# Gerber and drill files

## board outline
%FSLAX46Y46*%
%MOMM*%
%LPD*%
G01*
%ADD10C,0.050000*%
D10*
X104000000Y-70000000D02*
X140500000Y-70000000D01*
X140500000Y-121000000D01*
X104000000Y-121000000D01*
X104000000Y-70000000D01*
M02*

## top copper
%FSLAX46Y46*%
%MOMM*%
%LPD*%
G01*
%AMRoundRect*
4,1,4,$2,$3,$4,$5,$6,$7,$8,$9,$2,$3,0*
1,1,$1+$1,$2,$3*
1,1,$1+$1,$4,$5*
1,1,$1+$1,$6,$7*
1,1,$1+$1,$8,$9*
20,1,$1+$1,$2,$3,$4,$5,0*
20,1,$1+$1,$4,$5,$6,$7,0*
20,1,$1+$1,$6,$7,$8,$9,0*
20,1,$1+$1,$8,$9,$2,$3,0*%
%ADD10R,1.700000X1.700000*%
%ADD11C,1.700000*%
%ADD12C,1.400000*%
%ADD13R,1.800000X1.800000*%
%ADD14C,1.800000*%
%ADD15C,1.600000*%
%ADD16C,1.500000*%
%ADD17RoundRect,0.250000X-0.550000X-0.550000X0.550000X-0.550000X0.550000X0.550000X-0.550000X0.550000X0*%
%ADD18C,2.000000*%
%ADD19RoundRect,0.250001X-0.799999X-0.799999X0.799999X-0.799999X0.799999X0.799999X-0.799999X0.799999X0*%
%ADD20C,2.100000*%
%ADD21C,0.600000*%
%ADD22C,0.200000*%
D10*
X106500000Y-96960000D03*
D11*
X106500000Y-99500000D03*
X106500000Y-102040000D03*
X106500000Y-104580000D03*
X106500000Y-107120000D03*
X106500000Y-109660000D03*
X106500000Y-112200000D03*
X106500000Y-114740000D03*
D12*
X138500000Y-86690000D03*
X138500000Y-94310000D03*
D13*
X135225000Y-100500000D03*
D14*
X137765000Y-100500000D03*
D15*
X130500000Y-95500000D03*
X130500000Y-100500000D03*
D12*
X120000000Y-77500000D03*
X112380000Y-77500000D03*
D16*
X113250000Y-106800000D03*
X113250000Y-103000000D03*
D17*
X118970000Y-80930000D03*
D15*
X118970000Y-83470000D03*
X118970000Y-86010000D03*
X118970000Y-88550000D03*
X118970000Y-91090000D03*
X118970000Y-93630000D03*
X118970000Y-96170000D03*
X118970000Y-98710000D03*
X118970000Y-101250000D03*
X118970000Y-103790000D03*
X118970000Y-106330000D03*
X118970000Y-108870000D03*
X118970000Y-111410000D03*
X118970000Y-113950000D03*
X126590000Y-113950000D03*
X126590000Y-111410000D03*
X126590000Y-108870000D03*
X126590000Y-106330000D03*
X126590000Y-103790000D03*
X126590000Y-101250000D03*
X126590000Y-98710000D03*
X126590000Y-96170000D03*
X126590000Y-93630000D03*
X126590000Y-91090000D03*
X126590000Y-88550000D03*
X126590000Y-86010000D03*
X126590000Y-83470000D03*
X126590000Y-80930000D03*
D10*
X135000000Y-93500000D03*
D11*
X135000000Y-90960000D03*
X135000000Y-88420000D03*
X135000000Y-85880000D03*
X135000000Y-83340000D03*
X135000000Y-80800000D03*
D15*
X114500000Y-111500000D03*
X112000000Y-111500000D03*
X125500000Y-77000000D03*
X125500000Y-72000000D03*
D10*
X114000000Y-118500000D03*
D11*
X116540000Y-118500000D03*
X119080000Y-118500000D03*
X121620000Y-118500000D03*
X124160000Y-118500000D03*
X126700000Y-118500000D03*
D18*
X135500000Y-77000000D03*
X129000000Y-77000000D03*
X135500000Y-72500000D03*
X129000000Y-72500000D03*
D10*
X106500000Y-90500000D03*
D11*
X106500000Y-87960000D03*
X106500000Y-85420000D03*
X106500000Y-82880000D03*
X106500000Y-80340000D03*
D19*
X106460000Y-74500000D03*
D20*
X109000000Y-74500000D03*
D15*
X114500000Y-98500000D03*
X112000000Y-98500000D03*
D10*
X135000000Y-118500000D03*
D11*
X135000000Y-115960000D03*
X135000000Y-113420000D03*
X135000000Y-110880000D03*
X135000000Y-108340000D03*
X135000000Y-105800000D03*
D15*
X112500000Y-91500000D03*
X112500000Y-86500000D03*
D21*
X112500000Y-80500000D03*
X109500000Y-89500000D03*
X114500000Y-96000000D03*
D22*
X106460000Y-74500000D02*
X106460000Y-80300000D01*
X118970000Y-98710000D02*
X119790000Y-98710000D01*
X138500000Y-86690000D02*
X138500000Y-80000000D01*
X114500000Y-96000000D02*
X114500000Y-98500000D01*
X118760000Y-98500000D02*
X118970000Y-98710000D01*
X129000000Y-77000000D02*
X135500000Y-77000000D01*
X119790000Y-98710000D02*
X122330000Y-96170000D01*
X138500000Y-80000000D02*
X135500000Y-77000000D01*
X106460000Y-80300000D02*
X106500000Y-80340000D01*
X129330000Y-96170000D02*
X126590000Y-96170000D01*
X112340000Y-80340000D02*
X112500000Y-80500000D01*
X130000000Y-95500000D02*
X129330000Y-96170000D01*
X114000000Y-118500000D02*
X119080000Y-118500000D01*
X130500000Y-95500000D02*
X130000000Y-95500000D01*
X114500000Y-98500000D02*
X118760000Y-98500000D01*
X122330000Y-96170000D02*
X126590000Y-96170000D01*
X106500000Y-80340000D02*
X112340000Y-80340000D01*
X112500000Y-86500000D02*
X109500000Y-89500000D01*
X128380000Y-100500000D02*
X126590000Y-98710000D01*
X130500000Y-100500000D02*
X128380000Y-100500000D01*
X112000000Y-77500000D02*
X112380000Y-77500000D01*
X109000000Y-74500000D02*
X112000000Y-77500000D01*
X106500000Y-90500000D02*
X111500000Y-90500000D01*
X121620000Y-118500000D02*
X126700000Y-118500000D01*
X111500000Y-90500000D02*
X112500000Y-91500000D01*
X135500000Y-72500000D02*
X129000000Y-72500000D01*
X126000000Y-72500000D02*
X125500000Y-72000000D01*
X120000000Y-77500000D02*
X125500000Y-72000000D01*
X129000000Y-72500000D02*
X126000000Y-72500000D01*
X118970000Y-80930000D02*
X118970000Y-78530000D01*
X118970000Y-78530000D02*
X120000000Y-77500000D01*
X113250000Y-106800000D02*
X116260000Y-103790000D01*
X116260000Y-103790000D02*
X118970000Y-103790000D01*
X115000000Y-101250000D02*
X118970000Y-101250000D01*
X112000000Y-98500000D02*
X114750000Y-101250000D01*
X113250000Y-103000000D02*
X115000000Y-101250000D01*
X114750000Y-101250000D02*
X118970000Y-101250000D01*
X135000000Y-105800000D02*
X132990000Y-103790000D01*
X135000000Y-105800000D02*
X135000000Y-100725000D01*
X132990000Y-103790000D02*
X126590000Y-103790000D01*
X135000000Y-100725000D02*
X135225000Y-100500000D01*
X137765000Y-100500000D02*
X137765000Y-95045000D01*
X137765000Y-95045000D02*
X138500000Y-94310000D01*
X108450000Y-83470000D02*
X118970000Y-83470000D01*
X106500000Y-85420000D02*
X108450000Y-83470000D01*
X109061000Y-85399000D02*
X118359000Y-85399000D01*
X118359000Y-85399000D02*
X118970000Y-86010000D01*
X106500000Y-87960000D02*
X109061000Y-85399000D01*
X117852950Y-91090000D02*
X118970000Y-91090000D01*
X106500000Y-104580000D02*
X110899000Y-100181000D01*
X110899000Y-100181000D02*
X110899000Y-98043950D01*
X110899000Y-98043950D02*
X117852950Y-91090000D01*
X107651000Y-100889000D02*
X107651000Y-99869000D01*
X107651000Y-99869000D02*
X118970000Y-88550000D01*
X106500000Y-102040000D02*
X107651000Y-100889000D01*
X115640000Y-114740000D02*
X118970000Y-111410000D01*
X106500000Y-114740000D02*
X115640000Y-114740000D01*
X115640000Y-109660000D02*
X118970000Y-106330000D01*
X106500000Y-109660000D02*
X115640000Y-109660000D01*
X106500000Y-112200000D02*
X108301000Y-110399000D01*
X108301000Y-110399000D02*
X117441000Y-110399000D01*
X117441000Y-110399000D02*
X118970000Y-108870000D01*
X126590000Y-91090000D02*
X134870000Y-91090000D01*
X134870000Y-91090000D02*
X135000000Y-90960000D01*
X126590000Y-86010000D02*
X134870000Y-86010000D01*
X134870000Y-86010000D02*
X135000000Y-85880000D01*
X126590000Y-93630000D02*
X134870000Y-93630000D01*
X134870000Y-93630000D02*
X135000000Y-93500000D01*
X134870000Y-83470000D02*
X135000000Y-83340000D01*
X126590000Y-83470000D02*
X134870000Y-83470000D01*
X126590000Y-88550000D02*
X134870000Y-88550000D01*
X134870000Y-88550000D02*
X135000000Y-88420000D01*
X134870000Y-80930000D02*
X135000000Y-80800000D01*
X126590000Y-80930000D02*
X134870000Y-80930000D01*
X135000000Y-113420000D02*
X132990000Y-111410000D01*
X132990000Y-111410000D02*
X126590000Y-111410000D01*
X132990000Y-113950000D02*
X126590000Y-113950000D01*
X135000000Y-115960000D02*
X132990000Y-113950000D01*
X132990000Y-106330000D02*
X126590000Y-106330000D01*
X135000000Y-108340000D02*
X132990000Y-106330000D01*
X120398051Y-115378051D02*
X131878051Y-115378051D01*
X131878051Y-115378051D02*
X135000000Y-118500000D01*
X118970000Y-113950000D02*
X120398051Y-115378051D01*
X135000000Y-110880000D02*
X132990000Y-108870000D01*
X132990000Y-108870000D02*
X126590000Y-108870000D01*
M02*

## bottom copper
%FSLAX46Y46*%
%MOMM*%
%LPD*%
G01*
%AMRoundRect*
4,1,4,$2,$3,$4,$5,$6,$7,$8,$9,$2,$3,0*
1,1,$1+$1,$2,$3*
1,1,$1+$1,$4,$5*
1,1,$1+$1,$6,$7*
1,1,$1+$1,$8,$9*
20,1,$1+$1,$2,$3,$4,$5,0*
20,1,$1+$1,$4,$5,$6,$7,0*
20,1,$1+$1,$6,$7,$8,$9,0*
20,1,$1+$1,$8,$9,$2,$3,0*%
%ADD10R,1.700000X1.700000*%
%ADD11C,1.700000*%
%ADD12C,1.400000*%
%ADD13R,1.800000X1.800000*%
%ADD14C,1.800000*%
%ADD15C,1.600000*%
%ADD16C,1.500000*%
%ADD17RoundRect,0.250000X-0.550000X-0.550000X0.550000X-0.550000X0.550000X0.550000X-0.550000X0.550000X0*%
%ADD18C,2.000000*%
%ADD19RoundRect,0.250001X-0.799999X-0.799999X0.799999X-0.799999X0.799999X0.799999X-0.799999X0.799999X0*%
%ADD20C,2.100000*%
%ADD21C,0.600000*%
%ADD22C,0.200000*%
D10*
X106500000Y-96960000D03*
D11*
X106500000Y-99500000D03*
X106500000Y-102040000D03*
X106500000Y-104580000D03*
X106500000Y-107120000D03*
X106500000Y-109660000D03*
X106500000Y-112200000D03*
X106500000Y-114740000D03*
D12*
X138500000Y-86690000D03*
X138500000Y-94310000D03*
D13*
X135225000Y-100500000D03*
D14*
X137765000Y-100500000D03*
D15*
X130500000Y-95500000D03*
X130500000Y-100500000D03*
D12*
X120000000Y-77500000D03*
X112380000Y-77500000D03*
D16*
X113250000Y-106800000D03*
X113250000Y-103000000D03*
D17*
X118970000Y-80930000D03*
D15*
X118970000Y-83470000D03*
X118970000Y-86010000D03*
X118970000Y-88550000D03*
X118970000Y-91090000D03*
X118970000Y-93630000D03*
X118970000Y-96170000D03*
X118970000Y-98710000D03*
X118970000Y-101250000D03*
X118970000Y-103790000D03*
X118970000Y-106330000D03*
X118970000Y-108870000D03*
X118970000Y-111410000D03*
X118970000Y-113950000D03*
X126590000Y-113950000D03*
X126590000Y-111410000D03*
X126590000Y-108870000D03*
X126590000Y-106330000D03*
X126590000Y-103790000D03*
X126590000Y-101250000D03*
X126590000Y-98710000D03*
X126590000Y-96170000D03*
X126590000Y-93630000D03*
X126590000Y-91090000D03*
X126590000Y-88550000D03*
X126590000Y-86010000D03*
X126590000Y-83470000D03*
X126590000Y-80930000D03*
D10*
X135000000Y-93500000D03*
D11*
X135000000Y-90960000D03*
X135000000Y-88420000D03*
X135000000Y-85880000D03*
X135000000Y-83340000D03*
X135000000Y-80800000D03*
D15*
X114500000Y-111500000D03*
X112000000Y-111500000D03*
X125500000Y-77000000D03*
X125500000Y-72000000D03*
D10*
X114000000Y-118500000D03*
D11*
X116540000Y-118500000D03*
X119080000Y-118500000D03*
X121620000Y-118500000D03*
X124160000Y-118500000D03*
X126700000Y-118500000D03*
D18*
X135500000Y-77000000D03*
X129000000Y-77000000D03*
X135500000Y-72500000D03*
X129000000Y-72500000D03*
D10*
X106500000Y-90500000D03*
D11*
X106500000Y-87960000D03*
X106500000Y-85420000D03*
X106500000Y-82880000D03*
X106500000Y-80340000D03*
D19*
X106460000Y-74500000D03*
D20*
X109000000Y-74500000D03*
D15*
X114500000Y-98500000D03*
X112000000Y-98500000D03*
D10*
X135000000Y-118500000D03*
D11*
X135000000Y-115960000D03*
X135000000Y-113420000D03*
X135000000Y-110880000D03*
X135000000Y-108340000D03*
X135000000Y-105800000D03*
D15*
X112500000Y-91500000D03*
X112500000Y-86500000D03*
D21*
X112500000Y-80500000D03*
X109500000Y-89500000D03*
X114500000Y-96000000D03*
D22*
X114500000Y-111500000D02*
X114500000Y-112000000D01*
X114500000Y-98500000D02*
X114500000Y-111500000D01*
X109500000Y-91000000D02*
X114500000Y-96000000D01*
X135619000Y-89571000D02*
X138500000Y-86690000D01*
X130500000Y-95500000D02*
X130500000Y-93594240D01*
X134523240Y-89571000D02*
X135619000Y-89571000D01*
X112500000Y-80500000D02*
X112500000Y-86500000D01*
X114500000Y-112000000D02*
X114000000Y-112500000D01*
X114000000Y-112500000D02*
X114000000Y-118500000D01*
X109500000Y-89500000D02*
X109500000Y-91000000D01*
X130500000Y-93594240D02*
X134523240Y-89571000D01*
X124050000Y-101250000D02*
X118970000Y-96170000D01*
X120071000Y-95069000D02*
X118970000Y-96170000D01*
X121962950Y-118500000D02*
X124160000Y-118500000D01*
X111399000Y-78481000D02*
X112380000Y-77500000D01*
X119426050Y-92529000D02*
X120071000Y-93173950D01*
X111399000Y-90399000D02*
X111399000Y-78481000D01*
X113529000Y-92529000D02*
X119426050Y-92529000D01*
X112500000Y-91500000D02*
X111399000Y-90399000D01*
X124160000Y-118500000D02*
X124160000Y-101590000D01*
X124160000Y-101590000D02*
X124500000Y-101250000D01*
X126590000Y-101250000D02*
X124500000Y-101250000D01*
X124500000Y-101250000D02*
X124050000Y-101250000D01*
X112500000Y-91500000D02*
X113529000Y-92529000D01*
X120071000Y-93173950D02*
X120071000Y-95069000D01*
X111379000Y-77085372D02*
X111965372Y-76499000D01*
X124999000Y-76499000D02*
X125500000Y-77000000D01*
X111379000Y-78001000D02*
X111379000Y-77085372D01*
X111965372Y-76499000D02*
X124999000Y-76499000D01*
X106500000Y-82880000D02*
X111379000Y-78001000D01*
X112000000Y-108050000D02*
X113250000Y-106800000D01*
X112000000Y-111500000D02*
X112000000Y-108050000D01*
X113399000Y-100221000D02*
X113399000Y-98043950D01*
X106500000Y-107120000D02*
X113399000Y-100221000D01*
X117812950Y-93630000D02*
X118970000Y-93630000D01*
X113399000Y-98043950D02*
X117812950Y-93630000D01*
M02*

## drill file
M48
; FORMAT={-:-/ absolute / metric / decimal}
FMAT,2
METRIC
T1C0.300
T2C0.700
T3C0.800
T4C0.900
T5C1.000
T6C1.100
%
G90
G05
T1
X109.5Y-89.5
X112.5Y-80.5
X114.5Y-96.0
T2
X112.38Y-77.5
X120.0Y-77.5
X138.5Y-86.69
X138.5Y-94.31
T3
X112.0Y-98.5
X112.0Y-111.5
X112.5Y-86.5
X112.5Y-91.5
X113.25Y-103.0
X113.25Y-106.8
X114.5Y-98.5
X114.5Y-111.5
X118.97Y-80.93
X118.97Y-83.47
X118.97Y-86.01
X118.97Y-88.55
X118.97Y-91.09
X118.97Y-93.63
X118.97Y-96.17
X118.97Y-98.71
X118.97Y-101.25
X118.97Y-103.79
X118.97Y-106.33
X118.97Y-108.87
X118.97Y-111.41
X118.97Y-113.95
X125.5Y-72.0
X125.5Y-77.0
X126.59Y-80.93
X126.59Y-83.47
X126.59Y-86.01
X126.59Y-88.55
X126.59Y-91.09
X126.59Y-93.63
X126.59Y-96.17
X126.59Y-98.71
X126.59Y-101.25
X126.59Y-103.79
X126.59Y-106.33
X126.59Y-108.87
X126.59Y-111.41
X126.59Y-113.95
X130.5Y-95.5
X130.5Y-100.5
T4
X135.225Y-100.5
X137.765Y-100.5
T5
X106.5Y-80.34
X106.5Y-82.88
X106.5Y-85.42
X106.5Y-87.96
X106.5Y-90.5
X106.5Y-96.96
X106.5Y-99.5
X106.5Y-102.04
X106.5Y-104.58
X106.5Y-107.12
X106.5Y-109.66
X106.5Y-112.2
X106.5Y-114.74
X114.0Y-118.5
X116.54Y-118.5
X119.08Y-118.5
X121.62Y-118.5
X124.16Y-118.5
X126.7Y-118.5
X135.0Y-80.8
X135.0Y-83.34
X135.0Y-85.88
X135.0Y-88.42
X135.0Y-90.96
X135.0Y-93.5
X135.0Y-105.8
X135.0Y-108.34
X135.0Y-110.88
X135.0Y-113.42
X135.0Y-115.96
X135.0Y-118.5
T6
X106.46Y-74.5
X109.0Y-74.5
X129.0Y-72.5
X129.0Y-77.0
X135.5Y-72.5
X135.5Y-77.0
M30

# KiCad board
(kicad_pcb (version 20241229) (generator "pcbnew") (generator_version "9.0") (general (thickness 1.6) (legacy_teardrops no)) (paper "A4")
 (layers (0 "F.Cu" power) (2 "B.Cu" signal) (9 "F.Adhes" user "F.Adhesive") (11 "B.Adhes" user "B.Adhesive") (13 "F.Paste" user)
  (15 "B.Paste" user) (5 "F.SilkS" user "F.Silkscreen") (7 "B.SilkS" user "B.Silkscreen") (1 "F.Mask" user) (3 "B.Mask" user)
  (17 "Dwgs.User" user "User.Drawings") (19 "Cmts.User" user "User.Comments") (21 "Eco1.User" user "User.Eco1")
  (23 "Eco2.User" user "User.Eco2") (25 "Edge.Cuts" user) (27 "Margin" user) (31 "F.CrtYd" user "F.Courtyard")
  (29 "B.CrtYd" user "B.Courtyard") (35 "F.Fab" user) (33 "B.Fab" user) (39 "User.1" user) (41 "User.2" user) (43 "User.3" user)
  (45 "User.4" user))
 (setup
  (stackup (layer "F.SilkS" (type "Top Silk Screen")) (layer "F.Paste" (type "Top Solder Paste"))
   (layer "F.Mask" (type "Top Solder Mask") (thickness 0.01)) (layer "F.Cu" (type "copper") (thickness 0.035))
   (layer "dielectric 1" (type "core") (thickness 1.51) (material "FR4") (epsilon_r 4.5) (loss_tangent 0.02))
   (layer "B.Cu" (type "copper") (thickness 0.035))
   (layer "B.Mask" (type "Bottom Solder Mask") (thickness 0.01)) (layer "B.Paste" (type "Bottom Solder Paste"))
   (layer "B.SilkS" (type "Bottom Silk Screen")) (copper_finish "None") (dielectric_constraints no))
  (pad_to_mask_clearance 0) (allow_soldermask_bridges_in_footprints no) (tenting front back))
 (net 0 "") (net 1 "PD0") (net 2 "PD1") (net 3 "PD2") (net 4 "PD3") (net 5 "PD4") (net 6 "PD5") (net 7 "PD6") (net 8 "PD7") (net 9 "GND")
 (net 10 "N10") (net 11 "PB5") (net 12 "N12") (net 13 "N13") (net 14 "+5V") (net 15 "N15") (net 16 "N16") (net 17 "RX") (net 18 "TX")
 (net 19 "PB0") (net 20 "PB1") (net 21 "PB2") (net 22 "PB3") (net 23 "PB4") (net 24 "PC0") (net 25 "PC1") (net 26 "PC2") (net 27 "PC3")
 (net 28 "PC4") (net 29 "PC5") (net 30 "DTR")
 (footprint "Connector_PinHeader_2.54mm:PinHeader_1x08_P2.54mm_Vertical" (layer "F.Cu") (at 106.5 96.96)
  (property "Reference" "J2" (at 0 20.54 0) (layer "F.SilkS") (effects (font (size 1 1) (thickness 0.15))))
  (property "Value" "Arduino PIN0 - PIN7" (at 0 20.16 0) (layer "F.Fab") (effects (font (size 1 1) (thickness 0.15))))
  (pad "1" thru_hole rect (at 0 0) (size 1.7 1.7) (drill 1) (layers "*.Cu" "*.Mask") (remove_unused_layers no) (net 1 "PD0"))
  (pad "2" thru_hole circle (at 0 2.54) (size 1.7 1.7) (drill 1) (layers "*.Cu" "*.Mask") (remove_unused_layers no) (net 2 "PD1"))
  (pad "3" thru_hole circle (at 0 5.08) (size 1.7 1.7) (drill 1) (layers "*.Cu" "*.Mask") (remove_unused_layers no) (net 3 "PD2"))
  (pad "4" thru_hole circle (at 0 7.62) (size 1.7 1.7) (drill 1) (layers "*.Cu" "*.Mask") (remove_unused_layers no) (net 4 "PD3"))
  (pad "5" thru_hole circle (at 0 10.16) (size 1.7 1.7) (drill 1) (layers "*.Cu" "*.Mask") (remove_unused_layers no) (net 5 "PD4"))
  (pad "6" thru_hole circle (at 0 12.7) (size 1.7 1.7) (drill 1) (layers "*.Cu" "*.Mask") (remove_unused_layers no) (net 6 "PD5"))
  (pad "7" thru_hole circle (at 0 15.24) (size 1.7 1.7) (drill 1) (layers "*.Cu" "*.Mask") (remove_unused_layers no) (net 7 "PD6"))
  (pad "8" thru_hole circle (at 0 17.78) (size 1.7 1.7) (drill 1) (layers "*.Cu" "*.Mask") (remove_unused_layers no) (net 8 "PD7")))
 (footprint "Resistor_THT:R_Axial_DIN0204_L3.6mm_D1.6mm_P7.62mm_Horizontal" (layer "F.Cu") (at 138.5 86.69 -90)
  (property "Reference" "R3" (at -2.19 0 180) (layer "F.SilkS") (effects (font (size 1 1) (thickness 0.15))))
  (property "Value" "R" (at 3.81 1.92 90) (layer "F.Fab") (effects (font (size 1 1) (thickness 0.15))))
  (pad "1" thru_hole circle (at 0 0 270) (size 1.4 1.4) (drill 0.7) (layers "*.Cu" "*.Mask") (remove_unused_layers no) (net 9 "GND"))
  (pad "2" thru_hole circle (at 7.62 0 270) (size 1.4 1.4) (drill 0.7) (layers "*.Cu" "*.Mask") (remove_unused_layers no) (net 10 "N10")))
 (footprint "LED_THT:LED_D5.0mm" (layer "F.Cu") (at 135.225 100.5)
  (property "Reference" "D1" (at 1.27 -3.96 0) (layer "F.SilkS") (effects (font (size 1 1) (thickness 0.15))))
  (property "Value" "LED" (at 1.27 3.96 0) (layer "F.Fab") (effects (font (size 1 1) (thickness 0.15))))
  (pad "1" thru_hole rect (at 0 0) (size 1.8 1.8) (drill 0.9) (layers "*.Cu" "*.Mask") (remove_unused_layers no) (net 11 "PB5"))
  (pad "2" thru_hole circle (at 2.54 0) (size 1.8 1.8) (drill 0.9) (layers "*.Cu" "*.Mask") (remove_unused_layers no) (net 10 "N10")))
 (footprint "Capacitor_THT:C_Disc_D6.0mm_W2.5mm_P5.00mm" (layer "F.Cu") (at 130.5 95.5 -90)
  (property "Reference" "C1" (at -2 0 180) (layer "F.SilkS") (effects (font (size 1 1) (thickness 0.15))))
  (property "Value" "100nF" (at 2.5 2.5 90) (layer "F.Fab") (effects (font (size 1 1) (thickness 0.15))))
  (pad "1" thru_hole circle (at 0 0 270) (size 1.6 1.6) (drill 0.8) (layers "*.Cu" "*.Mask") (remove_unused_layers no) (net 9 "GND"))
  (pad "2" thru_hole circle (at 5 0 270) (size 1.6 1.6) (drill 0.8) (layers "*.Cu" "*.Mask") (remove_unused_layers no) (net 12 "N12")))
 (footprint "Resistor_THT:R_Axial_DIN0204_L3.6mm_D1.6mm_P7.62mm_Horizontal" (layer "F.Cu") (at 120 77.5 180)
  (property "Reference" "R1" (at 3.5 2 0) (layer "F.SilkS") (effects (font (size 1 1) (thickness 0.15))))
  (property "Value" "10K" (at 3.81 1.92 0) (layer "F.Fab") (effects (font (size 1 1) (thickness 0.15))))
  (pad "1" thru_hole circle (at 0 0 180) (size 1.4 1.4) (drill 0.7) (layers "*.Cu" "*.Mask") (remove_unused_layers no) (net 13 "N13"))
  (pad "2" thru_hole circle (at 7.62 0 180) (size 1.4 1.4) (drill 0.7) (layers "*.Cu" "*.Mask") (remove_unused_layers no) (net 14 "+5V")))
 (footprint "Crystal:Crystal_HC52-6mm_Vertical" (layer "F.Cu") (at 113.25 106.8 90)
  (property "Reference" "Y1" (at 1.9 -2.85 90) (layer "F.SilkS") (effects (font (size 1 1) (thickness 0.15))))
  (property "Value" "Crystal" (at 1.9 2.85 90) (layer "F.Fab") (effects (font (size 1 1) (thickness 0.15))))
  (pad "1" thru_hole circle (at 0 0 90) (size 1.5 1.5) (drill 0.8) (layers "*.Cu" "*.Mask") (remove_unused_layers no) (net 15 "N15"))
  (pad "2" thru_hole circle (at 3.8 0 90) (size 1.5 1.5) (drill 0.8) (layers "*.Cu" "*.Mask") (remove_unused_layers no) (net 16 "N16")))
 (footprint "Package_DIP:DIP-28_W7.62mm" (layer "F.Cu") (at 118.97 80.93)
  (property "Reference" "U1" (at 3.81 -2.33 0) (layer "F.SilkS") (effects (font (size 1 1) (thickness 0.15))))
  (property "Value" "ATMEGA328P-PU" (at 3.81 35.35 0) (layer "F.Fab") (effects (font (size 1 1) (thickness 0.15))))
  (pad "1" thru_hole roundrect (at 0 0) (size 1.6 1.6) (drill 0.8) (layers "*.Cu" "*.Mask") (remove_unused_layers no)
   (roundrect_rratio 0.15625) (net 13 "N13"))
  (pad "2" thru_hole circle (at 0 2.54) (size 1.6 1.6) (drill 0.8) (layers "*.Cu" "*.Mask") (remove_unused_layers no) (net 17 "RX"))
  (pad "3" thru_hole circle (at 0 5.08) (size 1.6 1.6) (drill 0.8) (layers "*.Cu" "*.Mask") (remove_unused_layers no) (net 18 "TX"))
  (pad "4" thru_hole circle (at 0 7.62) (size 1.6 1.6) (drill 0.8) (layers "*.Cu" "*.Mask") (remove_unused_layers no) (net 3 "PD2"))
  (pad "5" thru_hole circle (at 0 10.16) (size 1.6 1.6) (drill 0.8) (layers "*.Cu" "*.Mask") (remove_unused_layers no) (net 4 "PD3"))
  (pad "6" thru_hole circle (at 0 12.7) (size 1.6 1.6) (drill 0.8) (layers "*.Cu" "*.Mask") (remove_unused_layers no) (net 5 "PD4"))
  (pad "7" thru_hole circle (at 0 15.24) (size 1.6 1.6) (drill 0.8) (layers "*.Cu" "*.Mask") (remove_unused_layers no) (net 14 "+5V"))
  (pad "8" thru_hole circle (at 0 17.78) (size 1.6 1.6) (drill 0.8) (layers "*.Cu" "*.Mask") (remove_unused_layers no) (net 9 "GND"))
  (pad "9" thru_hole circle (at 0 20.32) (size 1.6 1.6) (drill 0.8) (layers "*.Cu" "*.Mask") (remove_unused_layers no) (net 16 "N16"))
  (pad "10" thru_hole circle (at 0 22.86) (size 1.6 1.6) (drill 0.8) (layers "*.Cu" "*.Mask") (remove_unused_layers no) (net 15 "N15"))
  (pad "11" thru_hole circle (at 0 25.4) (size 1.6 1.6) (drill 0.8) (layers "*.Cu" "*.Mask") (remove_unused_layers no) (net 6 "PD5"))
  (pad "12" thru_hole circle (at 0 27.94) (size 1.6 1.6) (drill 0.8) (layers "*.Cu" "*.Mask") (remove_unused_layers no) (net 7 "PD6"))
  (pad "13" thru_hole circle (at 0 30.48) (size 1.6 1.6) (drill 0.8) (layers "*.Cu" "*.Mask") (remove_unused_layers no) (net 8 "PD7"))
  (pad "14" thru_hole circle (at 0 33.02) (size 1.6 1.6) (drill 0.8) (layers "*.Cu" "*.Mask") (remove_unused_layers no) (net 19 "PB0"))
  (pad "15" thru_hole circle (at 7.62 33.02) (size 1.6 1.6) (drill 0.8) (layers "*.Cu" "*.Mask") (remove_unused_layers no) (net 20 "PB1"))
  (pad "16" thru_hole circle (at 7.62 30.48) (size 1.6 1.6) (drill 0.8) (layers "*.Cu" "*.Mask") (remove_unused_layers no) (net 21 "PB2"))
  (pad "17" thru_hole circle (at 7.62 27.94) (size 1.6 1.6) (drill 0.8) (layers "*.Cu" "*.Mask") (remove_unused_layers no) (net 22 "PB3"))
  (pad "18" thru_hole circle (at 7.62 25.4) (size 1.6 1.6) (drill 0.8) (layers "*.Cu" "*.Mask") (remove_unused_layers no) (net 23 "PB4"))
  (pad "19" thru_hole circle (at 7.62 22.86) (size 1.6 1.6) (drill 0.8) (layers "*.Cu" "*.Mask") (remove_unused_layers no) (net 11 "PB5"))
  (pad "20" thru_hole circle (at 7.62 20.32) (size 1.6 1.6) (drill 0.8) (layers "*.Cu" "*.Mask") (remove_unused_layers no) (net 14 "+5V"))
  (pad "21" thru_hole circle (at 7.62 17.78) (size 1.6 1.6) (drill 0.8) (layers "*.Cu" "*.Mask") (remove_unused_layers no) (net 12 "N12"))
  (pad "22" thru_hole circle (at 7.62 15.24) (size 1.6 1.6) (drill 0.8) (layers "*.Cu" "*.Mask") (remove_unused_layers no) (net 9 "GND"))
  (pad "23" thru_hole circle (at 7.62 12.7) (size 1.6 1.6) (drill 0.8) (layers "*.Cu" "*.Mask") (remove_unused_layers no) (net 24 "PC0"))
  (pad "24" thru_hole circle (at 7.62 10.16) (size 1.6 1.6) (drill 0.8) (layers "*.Cu" "*.Mask") (remove_unused_layers no) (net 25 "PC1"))
  (pad "25" thru_hole circle (at 7.62 7.62) (size 1.6 1.6) (drill 0.8) (layers "*.Cu" "*.Mask") (remove_unused_layers no) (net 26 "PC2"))
  (pad "26" thru_hole circle (at 7.62 5.08) (size 1.6 1.6) (drill 0.8) (layers "*.Cu" "*.Mask") (remove_unused_layers no) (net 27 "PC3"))
  (pad "27" thru_hole circle (at 7.62 2.54) (size 1.6 1.6) (drill 0.8) (layers "*.Cu" "*.Mask") (remove_unused_layers no) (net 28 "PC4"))
  (pad "28" thru_hole circle (at 7.62 0) (size 1.6 1.6) (drill 0.8) (layers "*.Cu" "*.Mask") (remove_unused_layers no) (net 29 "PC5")))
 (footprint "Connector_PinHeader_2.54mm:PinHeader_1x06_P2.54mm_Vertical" (layer "F.Cu") (at 135 93.5 180)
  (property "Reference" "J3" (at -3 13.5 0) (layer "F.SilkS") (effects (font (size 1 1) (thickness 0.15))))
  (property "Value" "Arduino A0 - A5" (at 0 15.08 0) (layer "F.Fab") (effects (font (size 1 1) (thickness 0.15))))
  (pad "1" thru_hole rect (at 0 0 180) (size 1.7 1.7) (drill 1) (layers "*.Cu" "*.Mask") (remove_unused_layers no) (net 24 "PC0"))
  (pad "2" thru_hole circle (at 0 2.54 180) (size 1.7 1.7) (drill 1) (layers "*.Cu" "*.Mask") (remove_unused_layers no) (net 25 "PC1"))
  (pad "3" thru_hole circle (at 0 5.08 180) (size 1.7 1.7) (drill 1) (layers "*.Cu" "*.Mask") (remove_unused_layers no) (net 26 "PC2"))
  (pad "4" thru_hole circle (at 0 7.62 180) (size 1.7 1.7) (drill 1) (layers "*.Cu" "*.Mask") (remove_unused_layers no) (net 27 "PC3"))
  (pad "5" thru_hole circle (at 0 10.16 180) (size 1.7 1.7) (drill 1) (layers "*.Cu" "*.Mask") (remove_unused_layers no) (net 28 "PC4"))
  (pad "6" thru_hole circle (at 0 12.7 180) (size 1.7 1.7) (drill 1) (layers "*.Cu" "*.Mask") (remove_unused_layers no) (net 29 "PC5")))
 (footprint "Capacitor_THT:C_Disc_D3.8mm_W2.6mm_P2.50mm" (layer "F.Cu") (at 114.5 111.5 180)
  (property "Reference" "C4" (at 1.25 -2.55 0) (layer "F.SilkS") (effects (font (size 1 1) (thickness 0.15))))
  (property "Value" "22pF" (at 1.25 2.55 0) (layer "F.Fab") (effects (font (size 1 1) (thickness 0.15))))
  (pad "1" thru_hole circle (at 0 0 180) (size 1.6 1.6) (drill 0.8) (layers "*.Cu" "*.Mask") (remove_unused_layers no) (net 9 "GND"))
  (pad "2" thru_hole circle (at 2.5 0 180) (size 1.6 1.6) (drill 0.8) (layers "*.Cu" "*.Mask") (remove_unused_layers no) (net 15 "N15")))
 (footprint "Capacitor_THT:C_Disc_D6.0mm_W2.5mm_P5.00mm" (layer "F.Cu") (at 125.5 77 90)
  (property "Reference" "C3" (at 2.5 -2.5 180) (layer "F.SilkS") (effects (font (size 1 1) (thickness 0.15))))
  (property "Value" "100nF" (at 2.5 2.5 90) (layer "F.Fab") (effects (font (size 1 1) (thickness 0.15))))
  (pad "1" thru_hole circle (at 0 0 90) (size 1.6 1.6) (drill 0.8) (layers "*.Cu" "*.Mask") (remove_unused_layers no) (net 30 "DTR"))
  (pad "2" thru_hole circle (at 5 0 90) (size 1.6 1.6) (drill 0.8) (layers "*.Cu" "*.Mask") (remove_unused_layers no) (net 13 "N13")))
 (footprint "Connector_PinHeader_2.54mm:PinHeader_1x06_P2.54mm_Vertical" (layer "F.Cu") (at 114 118.5 90)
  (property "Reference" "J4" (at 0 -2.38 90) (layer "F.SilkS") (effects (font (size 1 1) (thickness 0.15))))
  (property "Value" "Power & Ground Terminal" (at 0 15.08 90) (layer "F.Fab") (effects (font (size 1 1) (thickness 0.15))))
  (pad "1" thru_hole rect (at 0 0 90) (size 1.7 1.7) (drill 1) (layers "*.Cu" "*.Mask") (remove_unused_layers no) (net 9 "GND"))
  (pad "2" thru_hole circle (at 0 2.54 90) (size 1.7 1.7) (drill 1) (layers "*.Cu" "*.Mask") (remove_unused_layers no) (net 9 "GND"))
  (pad "3" thru_hole circle (at 0 5.08 90) (size 1.7 1.7) (drill 1) (layers "*.Cu" "*.Mask") (remove_unused_layers no) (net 9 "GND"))
  (pad "4" thru_hole circle (at 0 7.62 90) (size 1.7 1.7) (drill 1) (layers "*.Cu" "*.Mask") (remove_unused_layers no) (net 14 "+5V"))
  (pad "5" thru_hole circle (at 0 10.16 90) (size 1.7 1.7) (drill 1) (layers "*.Cu" "*.Mask") (remove_unused_layers no) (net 14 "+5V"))
  (pad "6" thru_hole circle (at 0 12.7 90) (size 1.7 1.7) (drill 1) (layers "*.Cu" "*.Mask") (remove_unused_layers no) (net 14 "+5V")))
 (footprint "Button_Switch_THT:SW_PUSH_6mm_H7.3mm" (layer "F.Cu") (at 135.5 77 180)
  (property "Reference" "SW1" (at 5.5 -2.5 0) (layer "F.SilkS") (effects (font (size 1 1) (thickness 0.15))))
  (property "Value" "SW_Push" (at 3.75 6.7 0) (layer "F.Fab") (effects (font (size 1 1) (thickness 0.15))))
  (pad "1" thru_hole circle (at 0 0 270) (size 2 2) (drill 1.1) (layers "*.Cu" "*.Mask") (remove_unused_layers no) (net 9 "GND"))
  (pad "1" thru_hole circle (at 6.5 0 270) (size 2 2) (drill 1.1) (layers "*.Cu" "*.Mask") (remove_unused_layers no) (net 9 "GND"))
  (pad "2" thru_hole circle (at 0 4.5 270) (size 2 2) (drill 1.1) (layers "*.Cu" "*.Mask") (remove_unused_layers no) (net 13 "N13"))
  (pad "2" thru_hole circle (at 6.5 4.5 270) (size 2 2) (drill 1.1) (layers "*.Cu" "*.Mask") (remove_unused_layers no) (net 13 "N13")))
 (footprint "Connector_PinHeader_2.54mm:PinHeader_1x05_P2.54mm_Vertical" (layer "F.Cu") (at 106.5 90.5 180)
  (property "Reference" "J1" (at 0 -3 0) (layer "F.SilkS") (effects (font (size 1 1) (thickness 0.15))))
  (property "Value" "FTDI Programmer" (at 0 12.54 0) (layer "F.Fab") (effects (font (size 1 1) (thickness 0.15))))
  (pad "1" thru_hole rect (at 0 0 180) (size 1.7 1.7) (drill 1) (layers "*.Cu" "*.Mask") (remove_unused_layers no) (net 14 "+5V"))
  (pad "2" thru_hole circle (at 0 2.54 180) (size 1.7 1.7) (drill 1) (layers "*.Cu" "*.Mask") (remove_unused_layers no) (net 18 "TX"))
  (pad "3" thru_hole circle (at 0 5.08 180) (size 1.7 1.7) (drill 1) (layers "*.Cu" "*.Mask") (remove_unused_layers no) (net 17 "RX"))
  (pad "4" thru_hole circle (at 0 7.62 180) (size 1.7 1.7) (drill 1) (layers "*.Cu" "*.Mask") (remove_unused_layers no) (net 30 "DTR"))
  (pad "5" thru_hole circle (at 0 10.16 180) (size 1.7 1.7) (drill 1) (layers "*.Cu" "*.Mask") (remove_unused_layers no) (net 9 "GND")))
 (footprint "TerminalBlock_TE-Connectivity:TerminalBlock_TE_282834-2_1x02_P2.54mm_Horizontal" (layer "F.Cu") (at 106.46 74.5)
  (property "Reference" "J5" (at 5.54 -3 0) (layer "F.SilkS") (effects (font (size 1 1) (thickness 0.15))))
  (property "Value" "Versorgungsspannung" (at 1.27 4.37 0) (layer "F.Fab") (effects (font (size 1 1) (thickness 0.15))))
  (pad "1" thru_hole roundrect (at 0 0) (size 2.1 2.1) (drill 1.1) (layers "*.Cu" "*.Mask") (remove_unused_layers no)
   (roundrect_rratio 0.119048) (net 9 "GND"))
  (pad "2" thru_hole circle (at 2.54 0) (size 2.1 2.1) (drill 1.1) (layers "*.Cu" "*.Mask") (remove_unused_layers no) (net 14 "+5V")))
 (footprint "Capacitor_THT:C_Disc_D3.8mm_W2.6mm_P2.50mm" (layer "F.Cu") (at 114.5 98.5 180)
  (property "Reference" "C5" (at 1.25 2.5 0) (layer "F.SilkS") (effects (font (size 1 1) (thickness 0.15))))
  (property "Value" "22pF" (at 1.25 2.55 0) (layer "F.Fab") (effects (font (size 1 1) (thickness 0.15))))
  (pad "1" thru_hole circle (at 0 0 180) (size 1.6 1.6) (drill 0.8) (layers "*.Cu" "*.Mask") (remove_unused_layers no) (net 9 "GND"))
  (pad "2" thru_hole circle (at 2.5 0 180) (size 1.6 1.6) (drill 0.8) (layers "*.Cu" "*.Mask") (remove_unused_layers no) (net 16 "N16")))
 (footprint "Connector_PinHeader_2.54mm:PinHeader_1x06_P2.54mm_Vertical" (layer "F.Cu") (at 135 118.5 180)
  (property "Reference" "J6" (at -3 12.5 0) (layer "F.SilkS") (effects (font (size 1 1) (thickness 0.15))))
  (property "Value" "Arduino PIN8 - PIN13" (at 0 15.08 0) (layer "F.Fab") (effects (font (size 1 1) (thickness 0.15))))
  (pad "1" thru_hole rect (at 0 0 180) (size 1.7 1.7) (drill 1) (layers "*.Cu" "*.Mask") (remove_unused_layers no) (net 19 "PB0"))
  (pad "2" thru_hole circle (at 0 2.54 180) (size 1.7 1.7) (drill 1) (layers "*.Cu" "*.Mask") (remove_unused_layers no) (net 20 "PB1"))
  (pad "3" thru_hole circle (at 0 5.08 180) (size 1.7 1.7) (drill 1) (layers "*.Cu" "*.Mask") (remove_unused_layers no) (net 21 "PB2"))
  (pad "4" thru_hole circle (at 0 7.62 180) (size 1.7 1.7) (drill 1) (layers "*.Cu" "*.Mask") (remove_unused_layers no) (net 22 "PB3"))
  (pad "5" thru_hole circle (at 0 10.16 180) (size 1.7 1.7) (drill 1) (layers "*.Cu" "*.Mask") (remove_unused_layers no) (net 23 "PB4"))
  (pad "6" thru_hole circle (at 0 12.7 180) (size 1.7 1.7) (drill 1) (layers "*.Cu" "*.Mask") (remove_unused_layers no) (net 11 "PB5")))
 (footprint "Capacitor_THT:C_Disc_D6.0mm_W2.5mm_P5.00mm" (layer "F.Cu") (at 112.5 91.5 90)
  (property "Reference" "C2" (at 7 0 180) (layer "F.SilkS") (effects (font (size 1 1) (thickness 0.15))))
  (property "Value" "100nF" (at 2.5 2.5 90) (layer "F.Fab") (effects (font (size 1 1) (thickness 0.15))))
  (pad "1" thru_hole circle (at 0 0 90) (size 1.6 1.6) (drill 0.8) (layers "*.Cu" "*.Mask") (remove_unused_layers no) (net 14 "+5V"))
  (pad "2" thru_hole circle (at 5 0 90) (size 1.6 1.6) (drill 0.8) (layers "*.Cu" "*.Mask") (remove_unused_layers no) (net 9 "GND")))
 (gr_rect (start 104 70) (end 140.5 121) (stroke (width 0.05) (type default)) (fill no) (layer "Edge.Cuts"))
 (segment (start 106.46 74.5) (end 106.46 80.3) (width 0.2) (layer "F.Cu") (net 9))
 (segment (start 118.97 98.71) (end 119.79 98.71) (width 0.2) (layer "F.Cu") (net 9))
 (segment (start 138.5 86.69) (end 138.5 80) (width 0.2) (layer "F.Cu") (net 9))
 (segment (start 114.5 96) (end 114.5 98.5) (width 0.2) (layer "F.Cu") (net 9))
 (segment (start 118.76 98.5) (end 118.97 98.71) (width 0.2) (layer "F.Cu") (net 9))
 (segment (start 129 77) (end 135.5 77) (width 0.2) (layer "F.Cu") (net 9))
 (segment (start 119.79 98.71) (end 122.33 96.17) (width 0.2) (layer "F.Cu") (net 9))
 (segment (start 138.5 80) (end 135.5 77) (width 0.2) (layer "F.Cu") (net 9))
 (segment (start 106.46 80.3) (end 106.5 80.34) (width 0.2) (layer "F.Cu") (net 9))
 (segment (start 129.33 96.17) (end 126.59 96.17) (width 0.2) (layer "F.Cu") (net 9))
 (segment (start 112.34 80.34) (end 112.5 80.5) (width 0.2) (layer "F.Cu") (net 9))
 (segment (start 130 95.5) (end 129.33 96.17) (width 0.2) (layer "F.Cu") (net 9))
 (segment (start 114 118.5) (end 119.08 118.5) (width 0.2) (layer "F.Cu") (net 9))
 (segment (start 130.5 95.5) (end 130 95.5) (width 0.2) (layer "F.Cu") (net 9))
 (segment (start 114.5 98.5) (end 118.76 98.5) (width 0.2) (layer "F.Cu") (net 9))
 (segment (start 122.33 96.17) (end 126.59 96.17) (width 0.2) (layer "F.Cu") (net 9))
 (segment (start 106.5 80.34) (end 112.34 80.34) (width 0.2) (layer "F.Cu") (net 9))
 (segment (start 112.5 86.5) (end 109.5 89.5) (width 0.2) (layer "F.Cu") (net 9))
 (via (at 112.5 80.5) (size 0.6) (drill 0.3) (layers "F.Cu" "B.Cu") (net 9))
 (via (at 109.5 89.5) (size 0.6) (drill 0.3) (layers "F.Cu" "B.Cu") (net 9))
 (via (at 114.5 96) (size 0.6) (drill 0.3) (layers "F.Cu" "B.Cu") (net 9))
 (segment (start 114.5 111.5) (end 114.5 112) (width 0.2) (layer "B.Cu") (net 9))
 (segment (start 114.5 98.5) (end 114.5 111.5) (width 0.2) (layer "B.Cu") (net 9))
 (segment (start 109.5 91) (end 114.5 96) (width 0.2) (layer "B.Cu") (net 9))
 (segment (start 135.619 89.571) (end 138.5 86.69) (width 0.2) (layer "B.Cu") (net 9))
 (segment (start 130.5 95.5) (end 130.5 93.59424) (width 0.2) (layer "B.Cu") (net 9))
 (segment (start 134.52324 89.571) (end 135.619 89.571) (width 0.2) (layer "B.Cu") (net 9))
 (segment (start 112.5 80.5) (end 112.5 86.5) (width 0.2) (layer "B.Cu") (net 9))
 (segment (start 114.5 112) (end 114 112.5) (width 0.2) (layer "B.Cu") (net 9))
 (segment (start 114 112.5) (end 114 118.5) (width 0.2) (layer "B.Cu") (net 9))
 (segment (start 109.5 89.5) (end 109.5 91) (width 0.2) (layer "B.Cu") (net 9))
 (segment (start 130.5 93.59424) (end 134.52324 89.571) (width 0.2) (layer "B.Cu") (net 9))
 (segment (start 128.38 100.5) (end 126.59 98.71) (width 0.2) (layer "F.Cu") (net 12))
 (segment (start 130.5 100.5) (end 128.38 100.5) (width 0.2) (layer "F.Cu") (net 12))
 (segment (start 112 77.5) (end 112.38 77.5) (width 0.2) (layer "F.Cu") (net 14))
 (segment (start 109 74.5) (end 112 77.5) (width 0.2) (layer "F.Cu") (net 14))
 (segment (start 106.5 90.5) (end 111.5 90.5) (width 0.2) (layer "F.Cu") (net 14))
 (segment (start 121.62 118.5) (end 126.7 118.5) (width 0.2) (layer "F.Cu") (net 14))
 (segment (start 111.5 90.5) (end 112.5 91.5) (width 0.2) (layer "F.Cu") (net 14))
 (segment (start 124.05 101.25) (end 118.97 96.17) (width 0.2) (layer "B.Cu") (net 14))
 (segment (start 120.071 95.069) (end 118.97 96.17) (width 0.2) (layer "B.Cu") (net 14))
 (segment (start 121.96295 118.5) (end 124.16 118.5) (width 0.2) (layer "B.Cu") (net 14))
 (segment (start 111.399 78.481) (end 112.38 77.5) (width 0.2) (layer "B.Cu") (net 14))
 (segment (start 119.42605 92.529) (end 120.071 93.17395) (width 0.2) (layer "B.Cu") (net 14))
 (segment (start 111.399 90.399) (end 111.399 78.481) (width 0.2) (layer "B.Cu") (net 14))
 (segment (start 113.529 92.529) (end 119.42605 92.529) (width 0.2) (layer "B.Cu") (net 14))
 (segment (start 112.5 91.5) (end 111.399 90.399) (width 0.2) (layer "B.Cu") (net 14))
 (segment (start 124.16 118.5) (end 124.16 101.59) (width 0.2) (layer "B.Cu") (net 14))
 (segment (start 124.16 101.59) (end 124.5 101.25) (width 0.2) (layer "B.Cu") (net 14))
 (segment (start 126.59 101.25) (end 124.5 101.25) (width 0.2) (layer "B.Cu") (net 14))
 (segment (start 124.5 101.25) (end 124.05 101.25) (width 0.2) (layer "B.Cu") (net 14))
 (segment (start 112.5 91.5) (end 113.529 92.529) (width 0.2) (layer "B.Cu") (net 14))
 (segment (start 120.071 93.17395) (end 120.071 95.069) (width 0.2) (layer "B.Cu") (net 14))
 (segment (start 111.379 77.085372) (end 111.965372 76.499) (width 0.2) (layer "B.Cu") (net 30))
 (segment (start 124.999 76.499) (end 125.5 77) (width 0.2) (layer "B.Cu") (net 30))
 (segment (start 111.379 78.001) (end 111.379 77.085372) (width 0.2) (layer "B.Cu") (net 30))
 (segment (start 111.965372 76.499) (end 124.999 76.499) (width 0.2) (layer "B.Cu") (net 30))
 (segment (start 106.5 82.88) (end 111.379 78.001) (width 0.2) (layer "B.Cu") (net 30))
 (segment (start 135.5 72.5) (end 129 72.5) (width 0.2) (layer "F.Cu") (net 13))
 (segment (start 126 72.5) (end 125.5 72) (width 0.2) (layer "F.Cu") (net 13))
 (segment (start 120 77.5) (end 125.5 72) (width 0.2) (layer "F.Cu") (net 13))
 (segment (start 129 72.5) (end 126 72.5) (width 0.2) (layer "F.Cu") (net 13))
 (segment (start 118.97 80.93) (end 118.97 78.53) (width 0.2) (layer "F.Cu") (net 13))
 (segment (start 118.97 78.53) (end 120 77.5) (width 0.2) (layer "F.Cu") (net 13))
 (segment (start 113.25 106.8) (end 116.26 103.79) (width 0.2) (layer "F.Cu") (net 15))
 (segment (start 116.26 103.79) (end 118.97 103.79) (width 0.2) (layer "F.Cu") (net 15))
 (segment (start 112 108.05) (end 113.25 106.8) (width 0.2) (layer "B.Cu") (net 15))
 (segment (start 112 111.5) (end 112 108.05) (width 0.2) (layer "B.Cu") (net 15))
 (segment (start 115 101.25) (end 118.97 101.25) (width 0.2) (layer "F.Cu") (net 16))
 (segment (start 112 98.5) (end 114.75 101.25) (width 0.2) (layer "F.Cu") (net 16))
 (segment (start 113.25 103) (end 115 101.25) (width 0.2) (layer "F.Cu") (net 16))
 (segment (start 114.75 101.25) (end 118.97 101.25) (width 0.2) (layer "F.Cu") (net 16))
 (segment (start 135 105.8) (end 132.99 103.79) (width 0.2) (layer "F.Cu") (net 11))
 (segment (start 135 105.8) (end 135 100.725) (width 0.2) (layer "F.Cu") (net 11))
 (segment (start 132.99 103.79) (end 126.59 103.79) (width 0.2) (layer "F.Cu") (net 11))
 (segment (start 135 100.725) (end 135.225 100.5) (width 0.2) (layer "F.Cu") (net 11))
 (segment (start 137.765 100.5) (end 137.765 95.045) (width 0.2) (layer "F.Cu") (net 10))
 (segment (start 137.765 95.045) (end 138.5 94.31) (width 0.2) (layer "F.Cu") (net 10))
 (segment (start 108.45 83.47) (end 118.97 83.47) (width 0.2) (layer "F.Cu") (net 17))
 (segment (start 106.5 85.42) (end 108.45 83.47) (width 0.2) (layer "F.Cu") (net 17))
 (segment (start 109.061 85.399) (end 118.359 85.399) (width 0.2) (layer "F.Cu") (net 18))
 (segment (start 118.359 85.399) (end 118.97 86.01) (width 0.2) (layer "F.Cu") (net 18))
 (segment (start 106.5 87.96) (end 109.061 85.399) (width 0.2) (layer "F.Cu") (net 18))
 (segment (start 117.85295 91.09) (end 118.97 91.09) (width 0.2) (layer "F.Cu") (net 4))
 (segment (start 106.5 104.58) (end 110.899 100.181) (width 0.2) (layer "F.Cu") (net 4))
 (segment (start 110.899 100.181) (end 110.899 98.04395) (width 0.2) (layer "F.Cu") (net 4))
 (segment (start 110.899 98.04395) (end 117.85295 91.09) (width 0.2) (layer "F.Cu") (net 4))
 (segment (start 107.651 100.889) (end 107.651 99.869) (width 0.2) (layer "F.Cu") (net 3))
 (segment (start 107.651 99.869) (end 118.97 88.55) (width 0.2) (layer "F.Cu") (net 3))
 (segment (start 106.5 102.04) (end 107.651 100.889) (width 0.2) (layer "F.Cu") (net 3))
 (segment (start 115.64 114.74) (end 118.97 111.41) (width 0.2) (layer "F.Cu") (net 8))
 (segment (start 106.5 114.74) (end 115.64 114.74) (width 0.2) (layer "F.Cu") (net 8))
 (segment (start 113.399 100.221) (end 113.399 98.04395) (width 0.2) (layer "B.Cu") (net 5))
 (segment (start 106.5 107.12) (end 113.399 100.221) (width 0.2) (layer "B.Cu") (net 5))
 (segment (start 117.81295 93.63) (end 118.97 93.63) (width 0.2) (layer "B.Cu") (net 5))
 (segment (start 113.399 98.04395) (end 117.81295 93.63) (width 0.2) (layer "B.Cu") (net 5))
 (segment (start 115.64 109.66) (end 118.97 106.33) (width 0.2) (layer "F.Cu") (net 6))
 (segment (start 106.5 109.66) (end 115.64 109.66) (width 0.2) (layer "F.Cu") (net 6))
 (segment (start 106.5 112.2) (end 108.301 110.399) (width 0.2) (layer "F.Cu") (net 7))
 (segment (start 108.301 110.399) (end 117.441 110.399) (width 0.2) (layer "F.Cu") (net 7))
 (segment (start 117.441 110.399) (end 118.97 108.87) (width 0.2) (layer "F.Cu") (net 7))
 (segment (start 126.59 91.09) (end 134.87 91.09) (width 0.2) (layer "F.Cu") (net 25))
 (segment (start 134.87 91.09) (end 135 90.96) (width 0.2) (layer "F.Cu") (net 25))
 (segment (start 126.59 86.01) (end 134.87 86.01) (width 0.2) (layer "F.Cu") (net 27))
 (segment (start 134.87 86.01) (end 135 85.88) (width 0.2) (layer "F.Cu") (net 27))
 (segment (start 126.59 93.63) (end 134.87 93.63) (width 0.2) (layer "F.Cu") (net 24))
 (segment (start 134.87 93.63) (end 135 93.5) (width 0.2) (layer "F.Cu") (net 24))
 (segment (start 134.87 83.47) (end 135 83.34) (width 0.2) (layer "F.Cu") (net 28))
 (segment (start 126.59 83.47) (end 134.87 83.47) (width 0.2) (layer "F.Cu") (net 28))
 (segment (start 126.59 88.55) (end 134.87 88.55) (width 0.2) (layer "F.Cu") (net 26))
 (segment (start 134.87 88.55) (end 135 88.42) (width 0.2) (layer "F.Cu") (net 26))
 (segment (start 134.87 80.93) (end 135 80.8) (width 0.2) (layer "F.Cu") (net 29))
 (segment (start 126.59 80.93) (end 134.87 80.93) (width 0.2) (layer "F.Cu") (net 29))
 (segment (start 135 113.42) (end 132.99 111.41) (width 0.2) (layer "F.Cu") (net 21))
 (segment (start 132.99 111.41) (end 126.59 111.41) (width 0.2) (layer "F.Cu") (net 21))
 (segment (start 132.99 113.95) (end 126.59 113.95) (width 0.2) (layer "F.Cu") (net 20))
 (segment (start 135 115.96) (end 132.99 113.95) (width 0.2) (layer "F.Cu") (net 20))
 (segment (start 132.99 106.33) (end 126.59 106.33) (width 0.2) (layer "F.Cu") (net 23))
 (segment (start 135 108.34) (end 132.99 106.33) (width 0.2) (layer "F.Cu") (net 23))
 (segment (start 120.398051 115.378051) (end 131.878051 115.378051) (width 0.2) (layer "F.Cu") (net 19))
 (segment (start 131.878051 115.378051) (end 135 118.5) (width 0.2) (layer "F.Cu") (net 19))
 (segment (start 118.97 113.95) (end 120.398051 115.378051) (width 0.2) (layer "F.Cu") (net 19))
 (segment (start 135 110.88) (end 132.99 108.87) (width 0.2) (layer "F.Cu") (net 22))
 (segment (start 132.99 108.87) (end 126.59 108.87) (width 0.2) (layer "F.Cu") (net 22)))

